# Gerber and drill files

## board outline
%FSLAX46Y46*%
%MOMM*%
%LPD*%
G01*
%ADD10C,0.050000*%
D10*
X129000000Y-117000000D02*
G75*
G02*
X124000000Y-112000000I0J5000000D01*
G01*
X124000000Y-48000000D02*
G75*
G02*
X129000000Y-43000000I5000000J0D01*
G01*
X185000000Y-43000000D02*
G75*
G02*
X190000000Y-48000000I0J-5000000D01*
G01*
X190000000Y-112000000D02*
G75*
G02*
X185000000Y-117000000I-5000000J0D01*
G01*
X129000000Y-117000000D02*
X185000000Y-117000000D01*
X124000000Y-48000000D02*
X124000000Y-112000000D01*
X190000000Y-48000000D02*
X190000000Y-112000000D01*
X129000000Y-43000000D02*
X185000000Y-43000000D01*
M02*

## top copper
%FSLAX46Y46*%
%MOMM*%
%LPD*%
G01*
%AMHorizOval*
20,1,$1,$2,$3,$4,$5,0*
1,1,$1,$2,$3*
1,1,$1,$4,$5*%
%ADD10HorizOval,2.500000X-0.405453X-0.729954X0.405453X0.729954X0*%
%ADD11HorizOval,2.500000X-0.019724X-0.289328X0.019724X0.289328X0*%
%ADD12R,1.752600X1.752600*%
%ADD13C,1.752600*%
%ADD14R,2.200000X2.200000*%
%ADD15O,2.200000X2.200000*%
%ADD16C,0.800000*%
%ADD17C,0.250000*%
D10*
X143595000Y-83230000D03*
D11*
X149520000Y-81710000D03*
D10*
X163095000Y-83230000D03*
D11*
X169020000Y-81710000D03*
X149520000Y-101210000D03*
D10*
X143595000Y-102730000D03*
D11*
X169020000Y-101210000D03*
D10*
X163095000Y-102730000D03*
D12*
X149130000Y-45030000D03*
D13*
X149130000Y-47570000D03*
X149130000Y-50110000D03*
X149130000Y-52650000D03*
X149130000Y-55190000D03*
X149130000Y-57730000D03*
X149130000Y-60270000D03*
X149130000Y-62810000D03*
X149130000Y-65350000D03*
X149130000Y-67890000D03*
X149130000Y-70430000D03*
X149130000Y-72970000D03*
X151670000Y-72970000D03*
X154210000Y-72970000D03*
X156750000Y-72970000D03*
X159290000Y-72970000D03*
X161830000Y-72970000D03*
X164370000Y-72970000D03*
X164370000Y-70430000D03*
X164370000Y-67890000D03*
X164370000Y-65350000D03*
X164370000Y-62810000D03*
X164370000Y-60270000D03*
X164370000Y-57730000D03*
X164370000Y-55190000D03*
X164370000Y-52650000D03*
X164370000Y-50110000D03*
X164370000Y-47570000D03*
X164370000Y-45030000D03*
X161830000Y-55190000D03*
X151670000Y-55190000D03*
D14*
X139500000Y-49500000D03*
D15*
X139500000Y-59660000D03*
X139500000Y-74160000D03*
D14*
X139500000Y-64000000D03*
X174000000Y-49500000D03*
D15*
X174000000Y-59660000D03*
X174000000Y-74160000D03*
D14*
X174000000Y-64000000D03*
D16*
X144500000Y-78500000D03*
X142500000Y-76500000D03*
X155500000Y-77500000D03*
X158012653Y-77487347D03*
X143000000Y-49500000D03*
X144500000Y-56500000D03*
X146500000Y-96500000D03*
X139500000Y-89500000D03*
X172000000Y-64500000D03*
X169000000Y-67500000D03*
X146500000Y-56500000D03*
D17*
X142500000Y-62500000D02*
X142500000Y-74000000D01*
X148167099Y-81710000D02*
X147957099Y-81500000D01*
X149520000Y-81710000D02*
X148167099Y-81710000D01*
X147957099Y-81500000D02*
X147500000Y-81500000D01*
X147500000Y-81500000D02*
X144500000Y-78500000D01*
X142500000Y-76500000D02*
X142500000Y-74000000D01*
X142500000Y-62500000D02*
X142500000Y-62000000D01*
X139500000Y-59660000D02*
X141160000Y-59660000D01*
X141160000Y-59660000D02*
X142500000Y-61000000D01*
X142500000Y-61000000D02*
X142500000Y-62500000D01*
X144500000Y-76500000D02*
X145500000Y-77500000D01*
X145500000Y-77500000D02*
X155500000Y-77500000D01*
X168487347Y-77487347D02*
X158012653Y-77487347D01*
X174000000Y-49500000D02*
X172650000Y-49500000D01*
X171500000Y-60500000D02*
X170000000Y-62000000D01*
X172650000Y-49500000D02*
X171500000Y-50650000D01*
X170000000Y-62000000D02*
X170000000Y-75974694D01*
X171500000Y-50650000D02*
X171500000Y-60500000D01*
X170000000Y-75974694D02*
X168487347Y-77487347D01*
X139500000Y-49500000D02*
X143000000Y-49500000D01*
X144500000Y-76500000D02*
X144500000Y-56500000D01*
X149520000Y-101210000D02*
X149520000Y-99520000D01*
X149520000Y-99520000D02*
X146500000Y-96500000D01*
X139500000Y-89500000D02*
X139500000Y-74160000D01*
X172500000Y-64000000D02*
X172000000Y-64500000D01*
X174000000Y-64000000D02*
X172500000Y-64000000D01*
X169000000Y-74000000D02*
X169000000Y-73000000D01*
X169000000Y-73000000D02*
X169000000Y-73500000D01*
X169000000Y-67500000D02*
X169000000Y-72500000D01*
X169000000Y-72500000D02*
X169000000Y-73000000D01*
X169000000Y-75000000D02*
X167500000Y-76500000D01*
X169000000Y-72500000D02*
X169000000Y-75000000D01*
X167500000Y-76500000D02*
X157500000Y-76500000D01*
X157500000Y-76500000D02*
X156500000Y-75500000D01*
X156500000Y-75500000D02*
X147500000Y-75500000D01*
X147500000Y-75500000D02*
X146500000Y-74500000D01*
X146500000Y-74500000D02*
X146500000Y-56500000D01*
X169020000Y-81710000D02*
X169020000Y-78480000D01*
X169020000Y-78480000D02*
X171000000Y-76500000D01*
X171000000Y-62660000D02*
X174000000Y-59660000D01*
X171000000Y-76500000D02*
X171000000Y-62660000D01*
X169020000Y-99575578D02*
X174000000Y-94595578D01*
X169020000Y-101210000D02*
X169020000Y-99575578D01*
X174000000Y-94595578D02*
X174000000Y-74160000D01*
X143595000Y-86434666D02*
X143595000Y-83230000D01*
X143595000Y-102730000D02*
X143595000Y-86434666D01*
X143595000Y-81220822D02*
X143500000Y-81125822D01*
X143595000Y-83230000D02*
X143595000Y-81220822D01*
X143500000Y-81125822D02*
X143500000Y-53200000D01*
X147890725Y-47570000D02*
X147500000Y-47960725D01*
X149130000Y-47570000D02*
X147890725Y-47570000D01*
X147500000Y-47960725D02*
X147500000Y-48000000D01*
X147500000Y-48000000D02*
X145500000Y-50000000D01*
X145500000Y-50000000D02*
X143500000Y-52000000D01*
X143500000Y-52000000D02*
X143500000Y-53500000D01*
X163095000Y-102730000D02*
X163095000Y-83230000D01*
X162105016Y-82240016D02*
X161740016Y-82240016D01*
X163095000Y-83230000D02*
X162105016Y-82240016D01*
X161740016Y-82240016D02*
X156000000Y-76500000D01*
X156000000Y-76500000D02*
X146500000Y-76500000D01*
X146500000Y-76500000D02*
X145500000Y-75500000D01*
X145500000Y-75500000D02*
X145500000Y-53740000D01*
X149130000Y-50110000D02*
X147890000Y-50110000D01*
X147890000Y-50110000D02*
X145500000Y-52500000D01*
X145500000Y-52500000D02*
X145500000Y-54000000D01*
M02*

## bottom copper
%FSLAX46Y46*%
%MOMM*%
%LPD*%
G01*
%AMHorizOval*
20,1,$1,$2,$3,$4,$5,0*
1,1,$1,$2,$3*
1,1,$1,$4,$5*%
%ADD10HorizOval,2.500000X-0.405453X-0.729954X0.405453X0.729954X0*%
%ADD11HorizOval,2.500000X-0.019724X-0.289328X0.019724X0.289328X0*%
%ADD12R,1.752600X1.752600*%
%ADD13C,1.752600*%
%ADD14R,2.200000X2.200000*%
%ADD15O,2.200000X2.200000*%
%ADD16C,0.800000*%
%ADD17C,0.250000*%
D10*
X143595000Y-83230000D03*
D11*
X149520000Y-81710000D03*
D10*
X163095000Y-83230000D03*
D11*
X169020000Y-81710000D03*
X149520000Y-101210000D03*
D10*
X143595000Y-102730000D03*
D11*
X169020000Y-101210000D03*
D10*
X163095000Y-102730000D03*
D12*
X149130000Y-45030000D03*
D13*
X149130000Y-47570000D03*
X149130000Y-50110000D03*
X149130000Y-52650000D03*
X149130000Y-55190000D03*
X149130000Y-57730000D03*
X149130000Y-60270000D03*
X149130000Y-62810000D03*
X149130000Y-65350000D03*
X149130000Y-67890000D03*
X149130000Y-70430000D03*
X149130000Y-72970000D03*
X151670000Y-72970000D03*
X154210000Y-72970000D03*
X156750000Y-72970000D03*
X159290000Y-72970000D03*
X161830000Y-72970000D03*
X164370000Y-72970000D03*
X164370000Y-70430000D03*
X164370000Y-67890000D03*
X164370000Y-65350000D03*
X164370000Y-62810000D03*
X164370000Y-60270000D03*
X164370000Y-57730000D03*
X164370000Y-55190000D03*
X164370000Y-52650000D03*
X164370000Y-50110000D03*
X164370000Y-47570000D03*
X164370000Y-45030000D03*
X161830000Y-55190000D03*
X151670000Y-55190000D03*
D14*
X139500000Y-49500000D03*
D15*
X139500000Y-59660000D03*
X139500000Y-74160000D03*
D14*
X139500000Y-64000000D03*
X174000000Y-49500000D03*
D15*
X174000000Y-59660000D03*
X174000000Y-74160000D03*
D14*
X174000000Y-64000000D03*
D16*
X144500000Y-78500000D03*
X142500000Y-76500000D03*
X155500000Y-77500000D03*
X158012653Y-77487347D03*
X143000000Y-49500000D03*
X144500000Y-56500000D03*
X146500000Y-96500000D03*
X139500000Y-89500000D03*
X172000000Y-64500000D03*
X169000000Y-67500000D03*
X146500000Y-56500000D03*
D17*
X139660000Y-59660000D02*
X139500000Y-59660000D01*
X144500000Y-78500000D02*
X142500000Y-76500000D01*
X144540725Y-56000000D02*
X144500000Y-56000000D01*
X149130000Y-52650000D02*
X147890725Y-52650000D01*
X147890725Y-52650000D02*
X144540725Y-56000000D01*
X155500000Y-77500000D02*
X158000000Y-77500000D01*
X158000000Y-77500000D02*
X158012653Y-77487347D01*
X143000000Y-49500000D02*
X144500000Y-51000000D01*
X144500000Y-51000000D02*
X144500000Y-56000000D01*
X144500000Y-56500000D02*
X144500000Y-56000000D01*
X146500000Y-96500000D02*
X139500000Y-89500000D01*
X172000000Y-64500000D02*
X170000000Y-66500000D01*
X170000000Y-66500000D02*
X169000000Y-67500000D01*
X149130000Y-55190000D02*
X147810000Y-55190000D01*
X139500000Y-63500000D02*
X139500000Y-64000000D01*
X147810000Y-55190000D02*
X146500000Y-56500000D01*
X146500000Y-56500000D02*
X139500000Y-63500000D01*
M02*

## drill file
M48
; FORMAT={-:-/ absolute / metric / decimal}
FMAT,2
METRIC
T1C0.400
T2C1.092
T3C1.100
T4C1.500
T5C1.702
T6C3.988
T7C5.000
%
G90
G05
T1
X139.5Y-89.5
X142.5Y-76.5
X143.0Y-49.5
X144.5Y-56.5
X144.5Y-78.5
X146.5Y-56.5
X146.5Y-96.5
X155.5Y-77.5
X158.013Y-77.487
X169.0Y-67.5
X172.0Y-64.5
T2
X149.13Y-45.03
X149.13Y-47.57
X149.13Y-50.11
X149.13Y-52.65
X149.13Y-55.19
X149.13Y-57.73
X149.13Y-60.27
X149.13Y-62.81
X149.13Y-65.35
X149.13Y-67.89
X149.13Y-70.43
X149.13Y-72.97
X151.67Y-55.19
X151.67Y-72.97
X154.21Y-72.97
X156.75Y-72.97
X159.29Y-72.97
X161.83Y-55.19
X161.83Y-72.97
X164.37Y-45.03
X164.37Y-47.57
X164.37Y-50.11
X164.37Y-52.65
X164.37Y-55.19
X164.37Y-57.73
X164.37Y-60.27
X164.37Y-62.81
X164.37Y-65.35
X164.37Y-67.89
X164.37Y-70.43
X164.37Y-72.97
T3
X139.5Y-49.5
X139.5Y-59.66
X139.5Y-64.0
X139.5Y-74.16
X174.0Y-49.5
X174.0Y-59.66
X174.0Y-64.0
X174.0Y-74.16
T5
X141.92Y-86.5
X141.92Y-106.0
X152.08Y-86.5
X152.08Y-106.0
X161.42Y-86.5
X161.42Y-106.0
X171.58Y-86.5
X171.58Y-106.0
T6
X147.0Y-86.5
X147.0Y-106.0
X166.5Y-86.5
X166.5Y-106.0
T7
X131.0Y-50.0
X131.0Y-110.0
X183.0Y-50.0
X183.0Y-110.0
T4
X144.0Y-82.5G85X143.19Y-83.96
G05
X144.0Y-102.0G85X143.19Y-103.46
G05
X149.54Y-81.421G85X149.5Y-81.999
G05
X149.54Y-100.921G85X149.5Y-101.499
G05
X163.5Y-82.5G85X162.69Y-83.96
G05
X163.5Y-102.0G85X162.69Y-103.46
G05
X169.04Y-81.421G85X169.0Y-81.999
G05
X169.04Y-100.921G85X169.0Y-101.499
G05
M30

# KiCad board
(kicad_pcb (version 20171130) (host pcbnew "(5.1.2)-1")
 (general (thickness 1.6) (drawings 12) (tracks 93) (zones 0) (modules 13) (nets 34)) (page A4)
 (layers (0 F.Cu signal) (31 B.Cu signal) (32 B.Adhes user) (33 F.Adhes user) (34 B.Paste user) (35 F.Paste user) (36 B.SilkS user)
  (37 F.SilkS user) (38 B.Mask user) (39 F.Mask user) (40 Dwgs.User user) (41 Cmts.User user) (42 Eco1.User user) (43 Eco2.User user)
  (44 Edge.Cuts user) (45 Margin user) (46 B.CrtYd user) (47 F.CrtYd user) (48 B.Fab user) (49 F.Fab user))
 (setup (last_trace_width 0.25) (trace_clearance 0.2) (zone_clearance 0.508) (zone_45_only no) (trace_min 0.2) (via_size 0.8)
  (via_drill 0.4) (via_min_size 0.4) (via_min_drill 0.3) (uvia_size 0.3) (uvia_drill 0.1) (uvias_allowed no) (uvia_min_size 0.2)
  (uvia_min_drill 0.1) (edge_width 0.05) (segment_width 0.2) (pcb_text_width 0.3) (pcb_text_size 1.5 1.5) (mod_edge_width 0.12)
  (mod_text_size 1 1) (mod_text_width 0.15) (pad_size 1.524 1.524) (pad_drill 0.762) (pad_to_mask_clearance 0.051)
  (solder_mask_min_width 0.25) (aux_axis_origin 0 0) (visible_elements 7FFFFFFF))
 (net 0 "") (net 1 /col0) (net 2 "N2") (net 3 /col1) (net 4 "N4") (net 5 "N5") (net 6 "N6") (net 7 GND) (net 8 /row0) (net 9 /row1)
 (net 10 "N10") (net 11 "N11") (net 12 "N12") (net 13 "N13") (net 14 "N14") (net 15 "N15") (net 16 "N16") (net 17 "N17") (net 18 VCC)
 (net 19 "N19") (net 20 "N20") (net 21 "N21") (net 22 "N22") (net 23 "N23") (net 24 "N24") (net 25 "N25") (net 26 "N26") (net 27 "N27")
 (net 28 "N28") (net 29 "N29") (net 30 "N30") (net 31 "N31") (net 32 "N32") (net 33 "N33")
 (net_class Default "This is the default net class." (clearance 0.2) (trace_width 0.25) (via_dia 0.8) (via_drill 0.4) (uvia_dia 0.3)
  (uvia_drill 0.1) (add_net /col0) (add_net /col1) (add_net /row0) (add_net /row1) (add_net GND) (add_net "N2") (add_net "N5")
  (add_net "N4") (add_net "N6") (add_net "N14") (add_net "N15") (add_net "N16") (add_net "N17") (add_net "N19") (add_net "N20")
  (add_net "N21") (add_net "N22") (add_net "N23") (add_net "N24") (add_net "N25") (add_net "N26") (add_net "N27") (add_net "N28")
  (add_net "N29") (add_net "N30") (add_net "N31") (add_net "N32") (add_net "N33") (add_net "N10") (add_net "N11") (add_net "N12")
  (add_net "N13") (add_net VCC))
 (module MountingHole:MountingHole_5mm (layer F.Cu) (at 183 110)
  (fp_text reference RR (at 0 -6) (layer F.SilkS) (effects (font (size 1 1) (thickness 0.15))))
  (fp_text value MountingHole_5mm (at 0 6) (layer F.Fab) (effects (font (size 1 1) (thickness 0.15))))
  (pad 1 np_thru_hole circle (at 0 0) (size 5 5) (drill 5) (layers *.Cu *.Mask)))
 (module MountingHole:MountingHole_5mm (layer F.Cu) (at 131 110)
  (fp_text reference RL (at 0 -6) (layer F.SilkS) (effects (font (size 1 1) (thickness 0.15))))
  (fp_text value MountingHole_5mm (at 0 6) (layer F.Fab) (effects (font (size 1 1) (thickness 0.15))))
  (pad 1 np_thru_hole circle (at 0 0) (size 5 5) (drill 5) (layers *.Cu *.Mask)))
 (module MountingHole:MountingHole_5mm (layer F.Cu) (at 183 50)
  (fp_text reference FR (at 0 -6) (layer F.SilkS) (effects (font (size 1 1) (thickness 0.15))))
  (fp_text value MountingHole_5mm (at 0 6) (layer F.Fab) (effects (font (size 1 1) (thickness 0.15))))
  (pad 1 np_thru_hole circle (at 0 0) (size 5 5) (drill 5) (layers *.Cu *.Mask)))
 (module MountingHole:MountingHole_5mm (layer F.Cu) (at 131 50)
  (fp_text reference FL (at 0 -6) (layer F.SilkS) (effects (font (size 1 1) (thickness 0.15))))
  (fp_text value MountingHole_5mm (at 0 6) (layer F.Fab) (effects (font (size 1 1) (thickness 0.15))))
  (pad 1 np_thru_hole circle (at 0 0) (size 5 5) (drill 5) (layers *.Cu *.Mask)))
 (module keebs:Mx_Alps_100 (layer F.Cu) (at 147 86.5)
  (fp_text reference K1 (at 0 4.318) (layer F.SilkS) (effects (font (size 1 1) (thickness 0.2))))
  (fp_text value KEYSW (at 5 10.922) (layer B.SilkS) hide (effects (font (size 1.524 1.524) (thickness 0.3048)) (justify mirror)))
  (pad HOLE np_thru_hole circle (at 0 0) (size 3.9878 3.9878) (drill 3.9878) (layers *.Cu))
  (pad HOLE np_thru_hole circle (at -5.08 0) (size 1.7018 1.7018) (drill 1.7018) (layers *.Cu))
  (pad HOLE np_thru_hole circle (at 5.08 0) (size 1.7018 1.7018) (drill 1.7018) (layers *.Cu))
  (pad 1 thru_hole oval (at -3.405 -3.27 330.95) (size 2.5 4.17) (drill oval 1.5 3.17) (layers *.Cu *.Mask F.SilkS) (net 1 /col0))
  (pad 2 thru_hole oval (at 2.52 -4.79 356.1) (size 2.5 3.08) (drill oval 1.5 2.08) (layers *.Cu *.Mask F.SilkS) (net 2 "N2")))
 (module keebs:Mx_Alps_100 (layer F.Cu) (at 166.5 86.5)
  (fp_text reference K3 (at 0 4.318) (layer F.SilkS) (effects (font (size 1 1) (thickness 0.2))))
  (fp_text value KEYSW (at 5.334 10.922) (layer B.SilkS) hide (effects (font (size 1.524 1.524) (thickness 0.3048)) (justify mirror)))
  (pad HOLE np_thru_hole circle (at 0 0) (size 3.9878 3.9878) (drill 3.9878) (layers *.Cu))
  (pad HOLE np_thru_hole circle (at -5.08 0) (size 1.7018 1.7018) (drill 1.7018) (layers *.Cu))
  (pad HOLE np_thru_hole circle (at 5.08 0) (size 1.7018 1.7018) (drill 1.7018) (layers *.Cu))
  (pad 1 thru_hole oval (at -3.405 -3.27 330.95) (size 2.5 4.17) (drill oval 1.5 3.17) (layers *.Cu *.Mask F.SilkS) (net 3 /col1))
  (pad 2 thru_hole oval (at 2.52 -4.79 356.1) (size 2.5 3.08) (drill oval 1.5 2.08) (layers *.Cu *.Mask F.SilkS) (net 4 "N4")))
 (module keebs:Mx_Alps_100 (layer F.Cu) (at 147 106)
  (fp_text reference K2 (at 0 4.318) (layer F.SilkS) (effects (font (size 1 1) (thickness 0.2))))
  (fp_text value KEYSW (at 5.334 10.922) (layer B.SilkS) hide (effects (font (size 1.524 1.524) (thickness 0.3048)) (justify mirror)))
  (pad 2 thru_hole oval (at 2.52 -4.79 356.1) (size 2.5 3.08) (drill oval 1.5 2.08) (layers *.Cu *.Mask F.SilkS) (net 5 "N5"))
  (pad 1 thru_hole oval (at -3.405 -3.27 330.95) (size 2.5 4.17) (drill oval 1.5 3.17) (layers *.Cu *.Mask F.SilkS) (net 1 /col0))
  (pad HOLE np_thru_hole circle (at 5.08 0) (size 1.7018 1.7018) (drill 1.7018) (layers *.Cu))
  (pad HOLE np_thru_hole circle (at -5.08 0) (size 1.7018 1.7018) (drill 1.7018) (layers *.Cu))
  (pad HOLE np_thru_hole circle (at 0 0) (size 3.9878 3.9878) (drill 3.9878) (layers *.Cu)))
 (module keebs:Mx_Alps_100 (layer F.Cu) (at 166.5 106)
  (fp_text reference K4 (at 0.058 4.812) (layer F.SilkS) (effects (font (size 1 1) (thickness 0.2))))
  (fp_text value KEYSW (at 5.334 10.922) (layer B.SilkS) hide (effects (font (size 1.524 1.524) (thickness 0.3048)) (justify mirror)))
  (pad 2 thru_hole oval (at 2.52 -4.79 356.1) (size 2.5 3.08) (drill oval 1.5 2.08) (layers *.Cu *.Mask F.SilkS) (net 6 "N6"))
  (pad 1 thru_hole oval (at -3.405 -3.27 330.95) (size 2.5 4.17) (drill oval 1.5 3.17) (layers *.Cu *.Mask F.SilkS) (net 3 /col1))
  (pad HOLE np_thru_hole circle (at 5.08 0) (size 1.7018 1.7018) (drill 1.7018) (layers *.Cu))
  (pad HOLE np_thru_hole circle (at -5.08 0) (size 1.7018 1.7018) (drill 1.7018) (layers *.Cu))
  (pad HOLE np_thru_hole circle (at 0 0) (size 3.9878 3.9878) (drill 3.9878) (layers *.Cu)))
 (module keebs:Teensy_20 (layer F.Cu) (at 156.75 59 270)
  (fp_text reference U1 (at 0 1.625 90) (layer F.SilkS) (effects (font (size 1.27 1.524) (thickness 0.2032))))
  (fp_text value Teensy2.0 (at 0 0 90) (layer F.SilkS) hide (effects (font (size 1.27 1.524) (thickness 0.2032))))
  (pad 1 thru_hole rect (at -13.97 7.62 270) (size 1.7526 1.7526) (drill 1.0922) (layers *.Cu *.SilkS *.Mask) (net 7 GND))
  (pad 2 thru_hole circle (at -11.43 7.62 270) (size 1.7526 1.7526) (drill 1.0922) (layers *.Cu *.SilkS *.Mask) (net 1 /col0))
  (pad 3 thru_hole circle (at -8.89 7.62 270) (size 1.7526 1.7526) (drill 1.0922) (layers *.Cu *.SilkS *.Mask) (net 3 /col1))
  (pad 4 thru_hole circle (at -6.35 7.62 270) (size 1.7526 1.7526) (drill 1.0922) (layers *.Cu *.SilkS *.Mask) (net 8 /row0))
  (pad 5 thru_hole circle (at -3.81 7.62 270) (size 1.7526 1.7526) (drill 1.0922) (layers *.Cu *.SilkS *.Mask) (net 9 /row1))
  (pad 6 thru_hole circle (at -1.27 7.62 270) (size 1.7526 1.7526) (drill 1.0922) (layers *.Cu *.SilkS *.Mask) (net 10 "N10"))
  (pad 7 thru_hole circle (at 1.27 7.62 270) (size 1.7526 1.7526) (drill 1.0922) (layers *.Cu *.SilkS *.Mask) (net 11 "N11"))
  (pad 8 thru_hole circle (at 3.81 7.62 270) (size 1.7526 1.7526) (drill 1.0922) (layers *.Cu *.SilkS *.Mask) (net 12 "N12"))
  (pad 9 thru_hole circle (at 6.35 7.62 270) (size 1.7526 1.7526) (drill 1.0922) (layers *.Cu *.SilkS *.Mask) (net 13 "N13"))
  (pad 10 thru_hole circle (at 8.89 7.62 270) (size 1.7526 1.7526) (drill 1.0922) (layers *.Cu *.SilkS *.Mask) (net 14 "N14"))
  (pad 11 thru_hole circle (at 11.43 7.62 270) (size 1.7526 1.7526) (drill 1.0922) (layers *.Cu *.SilkS *.Mask) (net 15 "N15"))
  (pad 12 thru_hole circle (at 13.97 7.62 270) (size 1.7526 1.7526) (drill 1.0922) (layers *.Cu *.SilkS *.Mask) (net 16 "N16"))
  (pad 13 thru_hole circle (at 13.97 5.08 180) (size 1.7526 1.7526) (drill 1.0922) (layers *.Cu *.SilkS *.Mask) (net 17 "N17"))
  (pad 14 thru_hole circle (at 13.97 2.54 180) (size 1.7526 1.7526) (drill 1.0922) (layers *.Cu *.SilkS *.Mask) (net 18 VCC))
  (pad 15 thru_hole circle (at 13.97 0 180) (size 1.7526 1.7526) (drill 1.0922) (layers *.Cu *.SilkS *.Mask) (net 7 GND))
  (pad 16 thru_hole circle (at 13.97 -2.54 180) (size 1.7526 1.7526) (drill 1.0922) (layers *.Cu *.SilkS *.Mask) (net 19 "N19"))
  (pad 17 thru_hole circle (at 13.97 -5.08 180) (size 1.7526 1.7526) (drill 1.0922) (layers *.Cu *.SilkS *.Mask) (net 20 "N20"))
  (pad 18 thru_hole circle (at 13.97 -7.62 270) (size 1.7526 1.7526) (drill 1.0922) (layers *.Cu *.SilkS *.Mask) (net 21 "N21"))
  (pad 19 thru_hole circle (at 11.43 -7.62 270) (size 1.7526 1.7526) (drill 1.0922) (layers *.Cu *.SilkS *.Mask) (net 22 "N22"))
  (pad 20 thru_hole circle (at 8.89 -7.62 270) (size 1.7526 1.7526) (drill 1.0922) (layers *.Cu *.SilkS *.Mask) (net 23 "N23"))
  (pad 21 thru_hole circle (at 6.35 -7.62 270) (size 1.7526 1.7526) (drill 1.0922) (layers *.Cu *.SilkS *.Mask) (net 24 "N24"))
  (pad 22 thru_hole circle (at 3.81 -7.62 270) (size 1.7526 1.7526) (drill 1.0922) (layers *.Cu *.SilkS *.Mask) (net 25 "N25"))
  (pad 23 thru_hole circle (at 1.27 -7.62 270) (size 1.7526 1.7526) (drill 1.0922) (layers *.Cu *.SilkS *.Mask) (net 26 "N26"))
  (pad 24 thru_hole circle (at -1.27 -7.62 270) (size 1.7526 1.7526) (drill 1.0922) (layers *.Cu *.SilkS *.Mask) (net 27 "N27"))
  (pad 25 thru_hole circle (at -3.81 -7.62 270) (size 1.7526 1.7526) (drill 1.0922) (layers *.Cu *.SilkS *.Mask) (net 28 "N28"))
  (pad 26 thru_hole circle (at -6.35 -7.62 270) (size 1.7526 1.7526) (drill 1.0922) (layers *.Cu *.SilkS *.Mask) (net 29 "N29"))
  (pad 27 thru_hole circle (at -8.89 -7.62 270) (size 1.7526 1.7526) (drill 1.0922) (layers *.Cu *.SilkS *.Mask) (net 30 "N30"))
  (pad 28 thru_hole circle (at -11.43 -7.62 270) (size 1.7526 1.7526) (drill 1.0922) (layers *.Cu *.SilkS *.Mask) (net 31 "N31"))
  (pad 29 thru_hole circle (at -13.97 -7.62 270) (size 1.7526 1.7526) (drill 1.0922) (layers *.Cu *.SilkS *.Mask) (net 18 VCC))
  (pad 30 thru_hole circle (at -3.81 -5.08 180) (size 1.7526 1.7526) (drill 1.0922) (layers *.Cu *.SilkS *.Mask) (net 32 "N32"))
  (pad 31 thru_hole circle (at -3.81 5.08 180) (size 1.7526 1.7526) (drill 1.0922) (layers *.Cu *.SilkS *.Mask) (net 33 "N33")))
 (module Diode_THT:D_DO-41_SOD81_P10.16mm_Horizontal (layer F.Cu) (at 139.5 49.5 270)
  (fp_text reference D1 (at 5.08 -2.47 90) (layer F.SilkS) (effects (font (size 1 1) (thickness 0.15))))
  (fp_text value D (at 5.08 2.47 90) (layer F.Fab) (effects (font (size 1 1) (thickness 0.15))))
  (pad 1 thru_hole rect (at 0 0 270) (size 2.2 2.2) (drill 1.1) (layers *.Cu *.Mask) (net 8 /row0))
  (pad 2 thru_hole oval (at 10.16 0 270) (size 2.2 2.2) (drill 1.1) (layers *.Cu *.Mask) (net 2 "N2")))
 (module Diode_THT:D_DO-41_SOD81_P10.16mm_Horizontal (layer F.Cu) (at 139.5 64 270)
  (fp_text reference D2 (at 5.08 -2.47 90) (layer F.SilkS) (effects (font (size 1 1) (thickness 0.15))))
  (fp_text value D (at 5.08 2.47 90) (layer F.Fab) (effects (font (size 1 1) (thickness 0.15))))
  (pad 2 thru_hole oval (at 10.16 0 270) (size 2.2 2.2) (drill 1.1) (layers *.Cu *.Mask) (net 5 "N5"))
  (pad 1 thru_hole rect (at 0 0 270) (size 2.2 2.2) (drill 1.1) (layers *.Cu *.Mask) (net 9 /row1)))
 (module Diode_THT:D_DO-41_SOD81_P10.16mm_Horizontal (layer F.Cu) (at 174 49.5 270)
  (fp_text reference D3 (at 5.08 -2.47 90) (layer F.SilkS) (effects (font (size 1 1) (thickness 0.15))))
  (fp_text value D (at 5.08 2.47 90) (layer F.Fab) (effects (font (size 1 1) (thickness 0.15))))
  (pad 1 thru_hole rect (at 0 0 270) (size 2.2 2.2) (drill 1.1) (layers *.Cu *.Mask) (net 8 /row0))
  (pad 2 thru_hole oval (at 10.16 0 270) (size 2.2 2.2) (drill 1.1) (layers *.Cu *.Mask) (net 4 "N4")))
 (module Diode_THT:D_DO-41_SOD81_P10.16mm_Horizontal (layer F.Cu) (at 174 64 270)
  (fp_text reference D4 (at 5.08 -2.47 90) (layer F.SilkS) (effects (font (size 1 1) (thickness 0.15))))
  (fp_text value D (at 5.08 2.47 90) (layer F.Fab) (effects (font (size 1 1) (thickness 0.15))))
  (pad 2 thru_hole oval (at 10.16 0 270) (size 2.2 2.2) (drill 1.1) (layers *.Cu *.Mask) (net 6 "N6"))
  (pad 1 thru_hole rect (at 0 0 270) (size 2.2 2.2) (drill 1.1) (layers *.Cu *.Mask) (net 9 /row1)))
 (gr_arc (start 129 112) (end 124 112) (angle -90) (layer Edge.Cuts) (width 0.05))
 (gr_arc (start 129 48) (end 129 43) (angle -90) (layer Edge.Cuts) (width 0.05))
 (gr_arc (start 185 48) (end 190 48) (angle -90) (layer Edge.Cuts) (width 0.05))
 (gr_arc (start 185 112) (end 185 117) (angle -90) (layer Edge.Cuts) (width 0.05))
 (gr_line (start 129 117) (end 185 117) (layer Edge.Cuts) (width 0.05))
 (gr_line (start 124 48) (end 124 112) (layer Edge.Cuts) (width 0.05))
 (gr_line (start 190 48) (end 190 112) (layer Edge.Cuts) (width 0.05))
 (gr_line (start 129 43) (end 185 43) (layer Edge.Cuts) (width 0.05))
 (segment (start 142.5 62.5) (end 142.5 74) (width 0.25) (layer F.Cu) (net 2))
 (segment (start 139.66 59.66) (end 139.5 59.66) (width 0.25) (layer B.Cu) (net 2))
 (segment (start 148.167099 81.71) (end 147.957099 81.5) (width 0.25) (layer F.Cu) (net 2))
 (segment (start 149.52 81.71) (end 148.167099 81.71) (width 0.25) (layer F.Cu) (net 2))
 (via (at 144.5 78.5) (size 0.8) (drill 0.4) (layers F.Cu B.Cu) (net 2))
 (segment (start 147.957099 81.5) (end 147.5 81.5) (width 0.25) (layer F.Cu) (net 2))
 (segment (start 147.5 81.5) (end 144.5 78.5) (width 0.25) (layer F.Cu) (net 2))
 (via (at 142.5 76.5) (size 0.8) (drill 0.4) (layers F.Cu B.Cu) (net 2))
 (segment (start 144.5 78.5) (end 142.5 76.5) (width 0.25) (layer B.Cu) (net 2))
 (segment (start 142.5 76.5) (end 142.5 74) (width 0.25) (layer F.Cu) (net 2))
 (segment (start 142.5 62.5) (end 142.5 62) (width 0.25) (layer F.Cu) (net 2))
 (segment (start 139.5 59.66) (end 141.16 59.66) (width 0.25) (layer F.Cu) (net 2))
 (segment (start 141.16 59.66) (end 142.5 61) (width 0.25) (layer F.Cu) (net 2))
 (segment (start 142.5 61) (end 142.5 62.5) (width 0.25) (layer F.Cu) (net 2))
 (segment (start 144.540725 56) (end 144.5 56) (width 0.25) (layer B.Cu) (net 8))
 (segment (start 149.13 52.65) (end 147.890725 52.65) (width 0.25) (layer B.Cu) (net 8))
 (segment (start 147.890725 52.65) (end 144.540725 56) (width 0.25) (layer B.Cu) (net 8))
 (via (at 155.5 77.5) (size 0.8) (drill 0.4) (layers F.Cu B.Cu) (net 8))
 (segment (start 144.5 76.5) (end 145.5 77.5) (width 0.25) (layer F.Cu) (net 8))
 (segment (start 145.5 77.5) (end 155.5 77.5) (width 0.25) (layer F.Cu) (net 8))
 (via (at 158.012653 77.487347) (size 0.8) (drill 0.4) (layers F.Cu B.Cu) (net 8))
 (segment (start 155.5 77.5) (end 158 77.5) (width 0.25) (layer B.Cu) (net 8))
 (segment (start 158 77.5) (end 158.012653 77.487347) (width 0.25) (layer B.Cu) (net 8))
 (segment (start 168.487347 77.487347) (end 158.012653 77.487347) (width 0.25) (layer F.Cu) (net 8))
 (segment (start 174 49.5) (end 172.65 49.5) (width 0.25) (layer F.Cu) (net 8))
 (segment (start 171.5 60.5) (end 170 62) (width 0.25) (layer F.Cu) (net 8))
 (segment (start 172.65 49.5) (end 171.5 50.65) (width 0.25) (layer F.Cu) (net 8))
 (segment (start 170 62) (end 170 75.974694) (width 0.25) (layer F.Cu) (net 8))
 (segment (start 171.5 50.65) (end 171.5 60.5) (width 0.25) (layer F.Cu) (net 8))
 (segment (start 170 75.974694) (end 168.487347 77.487347) (width 0.25) (layer F.Cu) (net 8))
 (via (at 143 49.5) (size 0.8) (drill 0.4) (layers F.Cu B.Cu) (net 8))
 (segment (start 139.5 49.5) (end 143 49.5) (width 0.25) (layer F.Cu) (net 8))
 (segment (start 143 49.5) (end 144.5 51) (width 0.25) (layer B.Cu) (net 8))
 (segment (start 144.5 51) (end 144.5 56) (width 0.25) (layer B.Cu) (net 8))
 (via (at 144.5 56.5) (size 0.8) (drill 0.4) (layers F.Cu B.Cu) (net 8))
 (segment (start 144.5 76.5) (end 144.5 56.5) (width 0.25) (layer F.Cu) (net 8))
 (segment (start 144.5 56.5) (end 144.5 56) (width 0.25) (layer B.Cu) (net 8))
 (via (at 146.5 96.5) (size 0.8) (drill 0.4) (layers F.Cu B.Cu) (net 5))
 (segment (start 149.52 101.21) (end 149.52 99.52) (width 0.25) (layer F.Cu) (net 5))
 (segment (start 149.52 99.52) (end 146.5 96.5) (width 0.25) (layer F.Cu) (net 5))
 (segment (start 146.5 96.5) (end 139.5 89.5) (width 0.25) (layer B.Cu) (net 5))
 (via (at 139.5 89.5) (size 0.8) (drill 0.4) (layers F.Cu B.Cu) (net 5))
 (segment (start 139.5 89.5) (end 139.5 74.16) (width 0.25) (layer F.Cu) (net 5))
 (via (at 172 64.5) (size 0.8) (drill 0.4) (layers F.Cu B.Cu) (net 9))
 (segment (start 172 64.5) (end 170 66.5) (width 0.25) (layer B.Cu) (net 9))
 (segment (start 172.5 64) (end 172 64.5) (width 0.25) (layer F.Cu) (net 9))
 (segment (start 174 64) (end 172.5 64) (width 0.25) (layer F.Cu) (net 9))
 (via (at 169 67.5) (size 0.8) (drill 0.4) (layers F.Cu B.Cu) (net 9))
 (segment (start 170 66.5) (end 169 67.5) (width 0.25) (layer B.Cu) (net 9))
 (segment (start 169 74) (end 169 73) (width 0.25) (layer F.Cu) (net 9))
 (segment (start 169 73) (end 169 73.5) (width 0.25) (layer F.Cu) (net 9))
 (segment (start 169 67.5) (end 169 72.5) (width 0.25) (layer F.Cu) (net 9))
 (segment (start 169 72.5) (end 169 73) (width 0.25) (layer F.Cu) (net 9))
 (segment (start 169 75) (end 167.5 76.5) (width 0.25) (layer F.Cu) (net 9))
 (segment (start 169 72.5) (end 169 75) (width 0.25) (layer F.Cu) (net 9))
 (segment (start 167.5 76.5) (end 157.5 76.5) (width 0.25) (layer F.Cu) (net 9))
 (segment (start 157.5 76.5) (end 156.5 75.5) (width 0.25) (layer F.Cu) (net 9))
 (segment (start 156.5 75.5) (end 147.5 75.5) (width 0.25) (layer F.Cu) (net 9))
 (segment (start 147.5 75.5) (end 146.5 74.5) (width 0.25) (layer F.Cu) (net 9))
 (segment (start 149.13 55.19) (end 147.81 55.19) (width 0.25) (layer B.Cu) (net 9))
 (segment (start 139.5 63.5) (end 139.5 64) (width 0.25) (layer B.Cu) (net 9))
 (via (at 146.5 56.5) (size 0.8) (drill 0.4) (layers F.Cu B.Cu) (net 9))
 (segment (start 146.5 74.5) (end 146.5 56.5) (width 0.25) (layer F.Cu) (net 9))
 (segment (start 147.81 55.19) (end 146.5 56.5) (width 0.25) (layer B.Cu) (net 9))
 (segment (start 146.5 56.5) (end 139.5 63.5) (width 0.25) (layer B.Cu) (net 9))
 (segment (start 169.02 81.71) (end 169.02 78.48) (width 0.25) (layer F.Cu) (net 4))
 (segment (start 169.02 78.48) (end 171 76.5) (width 0.25) (layer F.Cu) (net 4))
 (segment (start 171 62.66) (end 174 59.66) (width 0.25) (layer F.Cu) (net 4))
 (segment (start 171 76.5) (end 171 62.66) (width 0.25) (layer F.Cu) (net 4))
 (segment (start 169.02 99.575578) (end 174 94.595578) (width 0.25) (layer F.Cu) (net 6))
 (segment (start 169.02 101.21) (end 169.02 99.575578) (width 0.25) (layer F.Cu) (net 6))
 (segment (start 174 94.595578) (end 174 74.16) (width 0.25) (layer F.Cu) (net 6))
 (segment (start 143.595 86.434666) (end 143.595 83.23) (width 0.25) (layer F.Cu) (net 1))
 (segment (start 143.595 102.73) (end 143.595 86.434666) (width 0.25) (layer F.Cu) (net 1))
 (segment (start 143.595 81.220822) (end 143.5 81.125822) (width 0.25) (layer F.Cu) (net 1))
 (segment (start 143.595 83.23) (end 143.595 81.220822) (width 0.25) (layer F.Cu) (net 1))
 (segment (start 143.5 81.125822) (end 143.5 53.2) (width 0.25) (layer F.Cu) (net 1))
 (segment (start 147.890725 47.57) (end 147.5 47.960725) (width 0.25) (layer F.Cu) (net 1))
 (segment (start 149.13 47.57) (end 147.890725 47.57) (width 0.25) (layer F.Cu) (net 1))
 (segment (start 147.5 47.960725) (end 147.5 48) (width 0.25) (layer F.Cu) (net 1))
 (segment (start 147.5 48) (end 145.5 50) (width 0.25) (layer F.Cu) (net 1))
 (segment (start 145.5 50) (end 143.5 52) (width 0.25) (layer F.Cu) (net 1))
 (segment (start 143.5 52) (end 143.5 53.5) (width 0.25) (layer F.Cu) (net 1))
 (segment (start 163.095 102.73) (end 163.095 83.23) (width 0.25) (layer F.Cu) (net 3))
 (segment (start 162.105016 82.240016) (end 161.740016 82.240016) (width 0.25) (layer F.Cu) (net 3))
 (segment (start 163.095 83.23) (end 162.105016 82.240016) (width 0.25) (layer F.Cu) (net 3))
 (segment (start 161.740016 82.240016) (end 156 76.5) (width 0.25) (layer F.Cu) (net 3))
 (segment (start 156 76.5) (end 146.5 76.5) (width 0.25) (layer F.Cu) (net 3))
 (segment (start 146.5 76.5) (end 145.5 75.5) (width 0.25) (layer F.Cu) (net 3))
 (segment (start 145.5 75.5) (end 145.5 53.74) (width 0.25) (layer F.Cu) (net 3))
 (segment (start 149.13 50.11) (end 147.89 50.11) (width 0.25) (layer F.Cu) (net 3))
 (segment (start 147.89 50.11) (end 145.5 52.5) (width 0.25) (layer F.Cu) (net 3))
 (segment (start 145.5 52.5) (end 145.5 54) (width 0.25) (layer F.Cu) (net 3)))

